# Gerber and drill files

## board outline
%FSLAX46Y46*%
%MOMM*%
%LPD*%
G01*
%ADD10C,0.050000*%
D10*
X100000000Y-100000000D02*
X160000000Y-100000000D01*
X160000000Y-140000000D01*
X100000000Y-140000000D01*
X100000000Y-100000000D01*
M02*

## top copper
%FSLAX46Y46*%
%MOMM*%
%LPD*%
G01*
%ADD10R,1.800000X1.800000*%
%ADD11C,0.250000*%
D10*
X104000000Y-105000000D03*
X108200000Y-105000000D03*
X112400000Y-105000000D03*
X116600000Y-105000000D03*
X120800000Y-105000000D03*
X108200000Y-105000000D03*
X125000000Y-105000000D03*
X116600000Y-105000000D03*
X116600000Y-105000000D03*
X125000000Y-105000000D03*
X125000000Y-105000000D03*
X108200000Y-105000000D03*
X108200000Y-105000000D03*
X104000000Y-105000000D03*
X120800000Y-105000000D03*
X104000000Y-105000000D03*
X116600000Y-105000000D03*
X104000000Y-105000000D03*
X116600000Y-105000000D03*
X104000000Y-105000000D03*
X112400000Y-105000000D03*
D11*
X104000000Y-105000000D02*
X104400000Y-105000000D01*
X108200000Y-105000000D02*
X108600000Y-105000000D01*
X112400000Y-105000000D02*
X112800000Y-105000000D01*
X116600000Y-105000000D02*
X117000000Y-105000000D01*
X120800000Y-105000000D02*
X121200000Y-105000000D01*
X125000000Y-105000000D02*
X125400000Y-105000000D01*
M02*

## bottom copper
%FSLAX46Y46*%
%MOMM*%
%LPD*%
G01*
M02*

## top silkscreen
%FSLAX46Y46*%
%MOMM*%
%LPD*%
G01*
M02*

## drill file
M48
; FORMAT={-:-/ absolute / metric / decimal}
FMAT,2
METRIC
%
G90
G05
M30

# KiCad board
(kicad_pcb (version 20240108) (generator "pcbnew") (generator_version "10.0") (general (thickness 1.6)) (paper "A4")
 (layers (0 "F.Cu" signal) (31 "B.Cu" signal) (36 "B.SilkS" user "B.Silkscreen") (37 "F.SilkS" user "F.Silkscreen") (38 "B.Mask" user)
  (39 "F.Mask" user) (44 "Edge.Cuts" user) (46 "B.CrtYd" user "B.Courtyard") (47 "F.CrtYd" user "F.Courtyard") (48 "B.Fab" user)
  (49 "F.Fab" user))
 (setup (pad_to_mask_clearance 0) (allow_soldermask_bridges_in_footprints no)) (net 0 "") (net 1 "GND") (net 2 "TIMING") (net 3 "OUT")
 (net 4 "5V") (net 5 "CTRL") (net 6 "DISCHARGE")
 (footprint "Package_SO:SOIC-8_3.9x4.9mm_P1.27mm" (layer "F.Cu") (at 100 100)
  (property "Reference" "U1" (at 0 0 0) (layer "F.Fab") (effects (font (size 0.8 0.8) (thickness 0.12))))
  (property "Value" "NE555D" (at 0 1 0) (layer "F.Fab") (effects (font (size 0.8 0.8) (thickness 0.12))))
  (pad "1" smd rect (at 4.000 5.000) (size 1.8 1.8) (layers "F.Cu" "F.Paste" "F.Mask") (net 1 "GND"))
  (pad "2" smd rect (at 8.200 5.000) (size 1.8 1.8) (layers "F.Cu" "F.Paste" "F.Mask") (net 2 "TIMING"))
  (pad "3" smd rect (at 12.400 5.000) (size 1.8 1.8) (layers "F.Cu" "F.Paste" "F.Mask") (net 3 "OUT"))
  (pad "4" smd rect (at 16.600 5.000) (size 1.8 1.8) (layers "F.Cu" "F.Paste" "F.Mask") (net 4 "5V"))
  (pad "5" smd rect (at 20.800 5.000) (size 1.8 1.8) (layers "F.Cu" "F.Paste" "F.Mask") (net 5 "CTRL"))
  (pad "6" smd rect (at 8.200 5.000) (size 1.8 1.8) (layers "F.Cu" "F.Paste" "F.Mask") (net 2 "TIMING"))
  (pad "7" smd rect (at 25.000 5.000) (size 1.8 1.8) (layers "F.Cu" "F.Paste" "F.Mask") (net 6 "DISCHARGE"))
  (pad "8" smd rect (at 16.600 5.000) (size 1.8 1.8) (layers "F.Cu" "F.Paste" "F.Mask") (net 4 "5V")))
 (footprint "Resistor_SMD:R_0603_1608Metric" (layer "F.Cu") (at 100 100)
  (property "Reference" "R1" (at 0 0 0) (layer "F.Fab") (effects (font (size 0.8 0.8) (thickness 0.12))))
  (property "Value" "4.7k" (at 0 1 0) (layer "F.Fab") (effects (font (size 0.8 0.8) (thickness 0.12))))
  (pad "1" smd rect (at 16.600 5.000) (size 1.8 1.8) (layers "F.Cu" "F.Paste" "F.Mask") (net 4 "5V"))
  (pad "2" smd rect (at 25.000 5.000) (size 1.8 1.8) (layers "F.Cu" "F.Paste" "F.Mask") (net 6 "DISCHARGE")))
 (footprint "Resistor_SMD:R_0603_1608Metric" (layer "F.Cu") (at 100 100)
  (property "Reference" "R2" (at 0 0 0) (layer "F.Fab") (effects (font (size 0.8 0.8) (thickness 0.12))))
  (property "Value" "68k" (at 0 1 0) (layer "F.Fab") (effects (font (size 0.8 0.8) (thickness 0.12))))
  (pad "1" smd rect (at 25.000 5.000) (size 1.8 1.8) (layers "F.Cu" "F.Paste" "F.Mask") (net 6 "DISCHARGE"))
  (pad "2" smd rect (at 8.200 5.000) (size 1.8 1.8) (layers "F.Cu" "F.Paste" "F.Mask") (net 2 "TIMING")))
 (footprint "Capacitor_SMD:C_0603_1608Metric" (layer "F.Cu") (at 100 100)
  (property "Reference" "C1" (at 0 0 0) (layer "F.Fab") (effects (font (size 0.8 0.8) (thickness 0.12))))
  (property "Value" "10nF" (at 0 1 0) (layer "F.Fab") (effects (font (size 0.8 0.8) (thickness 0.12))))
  (pad "1" smd rect (at 8.200 5.000) (size 1.8 1.8) (layers "F.Cu" "F.Paste" "F.Mask") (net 2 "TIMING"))
  (pad "2" smd rect (at 4.000 5.000) (size 1.8 1.8) (layers "F.Cu" "F.Paste" "F.Mask") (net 1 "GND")))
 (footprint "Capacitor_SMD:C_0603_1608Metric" (layer "F.Cu") (at 100 100)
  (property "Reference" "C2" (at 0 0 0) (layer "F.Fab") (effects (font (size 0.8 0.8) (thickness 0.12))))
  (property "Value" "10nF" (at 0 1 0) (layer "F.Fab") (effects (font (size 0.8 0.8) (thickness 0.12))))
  (pad "1" smd rect (at 20.800 5.000) (size 1.8 1.8) (layers "F.Cu" "F.Paste" "F.Mask") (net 5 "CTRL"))
  (pad "2" smd rect (at 4.000 5.000) (size 1.8 1.8) (layers "F.Cu" "F.Paste" "F.Mask") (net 1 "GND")))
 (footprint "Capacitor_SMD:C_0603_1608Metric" (layer "F.Cu") (at 100 100)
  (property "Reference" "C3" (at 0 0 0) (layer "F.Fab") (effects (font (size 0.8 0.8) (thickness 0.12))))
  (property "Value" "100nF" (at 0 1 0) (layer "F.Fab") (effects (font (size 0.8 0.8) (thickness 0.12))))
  (pad "1" smd rect (at 16.600 5.000) (size 1.8 1.8) (layers "F.Cu" "F.Paste" "F.Mask") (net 4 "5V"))
  (pad "2" smd rect (at 4.000 5.000) (size 1.8 1.8) (layers "F.Cu" "F.Paste" "F.Mask") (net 1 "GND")))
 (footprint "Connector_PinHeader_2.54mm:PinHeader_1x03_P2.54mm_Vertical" (layer "F.Cu") (at 100 100)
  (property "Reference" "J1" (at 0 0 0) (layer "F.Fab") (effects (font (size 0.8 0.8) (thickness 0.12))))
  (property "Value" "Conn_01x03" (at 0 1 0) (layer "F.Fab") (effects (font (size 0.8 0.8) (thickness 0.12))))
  (pad "1" smd rect (at 16.600 5.000) (size 1.8 1.8) (layers "F.Cu" "F.Paste" "F.Mask") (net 4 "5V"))
  (pad "2" smd rect (at 4.000 5.000) (size 1.8 1.8) (layers "F.Cu" "F.Paste" "F.Mask") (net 1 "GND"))
  (pad "3" smd rect (at 12.400 5.000) (size 1.8 1.8) (layers "F.Cu" "F.Paste" "F.Mask") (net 3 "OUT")))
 (gr_rect (start 100 100) (end 160 140) (stroke (width 0.05) (type default)) (fill none) (layer "Edge.Cuts"))
 (segment (start 104.000 105.000) (end 104.400 105.000) (width 0.25) (layer "F.Cu") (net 1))
 (segment (start 108.200 105.000) (end 108.600 105.000) (width 0.25) (layer "F.Cu") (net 2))
 (segment (start 112.400 105.000) (end 112.800 105.000) (width 0.25) (layer "F.Cu") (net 3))
 (segment (start 116.600 105.000) (end 117.000 105.000) (width 0.25) (layer "F.Cu") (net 4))
 (segment (start 120.800 105.000) (end 121.200 105.000) (width 0.25) (layer "F.Cu") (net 5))
 (segment (start 125.000 105.000) (end 125.400 105.000) (width 0.25) (layer "F.Cu") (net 6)))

